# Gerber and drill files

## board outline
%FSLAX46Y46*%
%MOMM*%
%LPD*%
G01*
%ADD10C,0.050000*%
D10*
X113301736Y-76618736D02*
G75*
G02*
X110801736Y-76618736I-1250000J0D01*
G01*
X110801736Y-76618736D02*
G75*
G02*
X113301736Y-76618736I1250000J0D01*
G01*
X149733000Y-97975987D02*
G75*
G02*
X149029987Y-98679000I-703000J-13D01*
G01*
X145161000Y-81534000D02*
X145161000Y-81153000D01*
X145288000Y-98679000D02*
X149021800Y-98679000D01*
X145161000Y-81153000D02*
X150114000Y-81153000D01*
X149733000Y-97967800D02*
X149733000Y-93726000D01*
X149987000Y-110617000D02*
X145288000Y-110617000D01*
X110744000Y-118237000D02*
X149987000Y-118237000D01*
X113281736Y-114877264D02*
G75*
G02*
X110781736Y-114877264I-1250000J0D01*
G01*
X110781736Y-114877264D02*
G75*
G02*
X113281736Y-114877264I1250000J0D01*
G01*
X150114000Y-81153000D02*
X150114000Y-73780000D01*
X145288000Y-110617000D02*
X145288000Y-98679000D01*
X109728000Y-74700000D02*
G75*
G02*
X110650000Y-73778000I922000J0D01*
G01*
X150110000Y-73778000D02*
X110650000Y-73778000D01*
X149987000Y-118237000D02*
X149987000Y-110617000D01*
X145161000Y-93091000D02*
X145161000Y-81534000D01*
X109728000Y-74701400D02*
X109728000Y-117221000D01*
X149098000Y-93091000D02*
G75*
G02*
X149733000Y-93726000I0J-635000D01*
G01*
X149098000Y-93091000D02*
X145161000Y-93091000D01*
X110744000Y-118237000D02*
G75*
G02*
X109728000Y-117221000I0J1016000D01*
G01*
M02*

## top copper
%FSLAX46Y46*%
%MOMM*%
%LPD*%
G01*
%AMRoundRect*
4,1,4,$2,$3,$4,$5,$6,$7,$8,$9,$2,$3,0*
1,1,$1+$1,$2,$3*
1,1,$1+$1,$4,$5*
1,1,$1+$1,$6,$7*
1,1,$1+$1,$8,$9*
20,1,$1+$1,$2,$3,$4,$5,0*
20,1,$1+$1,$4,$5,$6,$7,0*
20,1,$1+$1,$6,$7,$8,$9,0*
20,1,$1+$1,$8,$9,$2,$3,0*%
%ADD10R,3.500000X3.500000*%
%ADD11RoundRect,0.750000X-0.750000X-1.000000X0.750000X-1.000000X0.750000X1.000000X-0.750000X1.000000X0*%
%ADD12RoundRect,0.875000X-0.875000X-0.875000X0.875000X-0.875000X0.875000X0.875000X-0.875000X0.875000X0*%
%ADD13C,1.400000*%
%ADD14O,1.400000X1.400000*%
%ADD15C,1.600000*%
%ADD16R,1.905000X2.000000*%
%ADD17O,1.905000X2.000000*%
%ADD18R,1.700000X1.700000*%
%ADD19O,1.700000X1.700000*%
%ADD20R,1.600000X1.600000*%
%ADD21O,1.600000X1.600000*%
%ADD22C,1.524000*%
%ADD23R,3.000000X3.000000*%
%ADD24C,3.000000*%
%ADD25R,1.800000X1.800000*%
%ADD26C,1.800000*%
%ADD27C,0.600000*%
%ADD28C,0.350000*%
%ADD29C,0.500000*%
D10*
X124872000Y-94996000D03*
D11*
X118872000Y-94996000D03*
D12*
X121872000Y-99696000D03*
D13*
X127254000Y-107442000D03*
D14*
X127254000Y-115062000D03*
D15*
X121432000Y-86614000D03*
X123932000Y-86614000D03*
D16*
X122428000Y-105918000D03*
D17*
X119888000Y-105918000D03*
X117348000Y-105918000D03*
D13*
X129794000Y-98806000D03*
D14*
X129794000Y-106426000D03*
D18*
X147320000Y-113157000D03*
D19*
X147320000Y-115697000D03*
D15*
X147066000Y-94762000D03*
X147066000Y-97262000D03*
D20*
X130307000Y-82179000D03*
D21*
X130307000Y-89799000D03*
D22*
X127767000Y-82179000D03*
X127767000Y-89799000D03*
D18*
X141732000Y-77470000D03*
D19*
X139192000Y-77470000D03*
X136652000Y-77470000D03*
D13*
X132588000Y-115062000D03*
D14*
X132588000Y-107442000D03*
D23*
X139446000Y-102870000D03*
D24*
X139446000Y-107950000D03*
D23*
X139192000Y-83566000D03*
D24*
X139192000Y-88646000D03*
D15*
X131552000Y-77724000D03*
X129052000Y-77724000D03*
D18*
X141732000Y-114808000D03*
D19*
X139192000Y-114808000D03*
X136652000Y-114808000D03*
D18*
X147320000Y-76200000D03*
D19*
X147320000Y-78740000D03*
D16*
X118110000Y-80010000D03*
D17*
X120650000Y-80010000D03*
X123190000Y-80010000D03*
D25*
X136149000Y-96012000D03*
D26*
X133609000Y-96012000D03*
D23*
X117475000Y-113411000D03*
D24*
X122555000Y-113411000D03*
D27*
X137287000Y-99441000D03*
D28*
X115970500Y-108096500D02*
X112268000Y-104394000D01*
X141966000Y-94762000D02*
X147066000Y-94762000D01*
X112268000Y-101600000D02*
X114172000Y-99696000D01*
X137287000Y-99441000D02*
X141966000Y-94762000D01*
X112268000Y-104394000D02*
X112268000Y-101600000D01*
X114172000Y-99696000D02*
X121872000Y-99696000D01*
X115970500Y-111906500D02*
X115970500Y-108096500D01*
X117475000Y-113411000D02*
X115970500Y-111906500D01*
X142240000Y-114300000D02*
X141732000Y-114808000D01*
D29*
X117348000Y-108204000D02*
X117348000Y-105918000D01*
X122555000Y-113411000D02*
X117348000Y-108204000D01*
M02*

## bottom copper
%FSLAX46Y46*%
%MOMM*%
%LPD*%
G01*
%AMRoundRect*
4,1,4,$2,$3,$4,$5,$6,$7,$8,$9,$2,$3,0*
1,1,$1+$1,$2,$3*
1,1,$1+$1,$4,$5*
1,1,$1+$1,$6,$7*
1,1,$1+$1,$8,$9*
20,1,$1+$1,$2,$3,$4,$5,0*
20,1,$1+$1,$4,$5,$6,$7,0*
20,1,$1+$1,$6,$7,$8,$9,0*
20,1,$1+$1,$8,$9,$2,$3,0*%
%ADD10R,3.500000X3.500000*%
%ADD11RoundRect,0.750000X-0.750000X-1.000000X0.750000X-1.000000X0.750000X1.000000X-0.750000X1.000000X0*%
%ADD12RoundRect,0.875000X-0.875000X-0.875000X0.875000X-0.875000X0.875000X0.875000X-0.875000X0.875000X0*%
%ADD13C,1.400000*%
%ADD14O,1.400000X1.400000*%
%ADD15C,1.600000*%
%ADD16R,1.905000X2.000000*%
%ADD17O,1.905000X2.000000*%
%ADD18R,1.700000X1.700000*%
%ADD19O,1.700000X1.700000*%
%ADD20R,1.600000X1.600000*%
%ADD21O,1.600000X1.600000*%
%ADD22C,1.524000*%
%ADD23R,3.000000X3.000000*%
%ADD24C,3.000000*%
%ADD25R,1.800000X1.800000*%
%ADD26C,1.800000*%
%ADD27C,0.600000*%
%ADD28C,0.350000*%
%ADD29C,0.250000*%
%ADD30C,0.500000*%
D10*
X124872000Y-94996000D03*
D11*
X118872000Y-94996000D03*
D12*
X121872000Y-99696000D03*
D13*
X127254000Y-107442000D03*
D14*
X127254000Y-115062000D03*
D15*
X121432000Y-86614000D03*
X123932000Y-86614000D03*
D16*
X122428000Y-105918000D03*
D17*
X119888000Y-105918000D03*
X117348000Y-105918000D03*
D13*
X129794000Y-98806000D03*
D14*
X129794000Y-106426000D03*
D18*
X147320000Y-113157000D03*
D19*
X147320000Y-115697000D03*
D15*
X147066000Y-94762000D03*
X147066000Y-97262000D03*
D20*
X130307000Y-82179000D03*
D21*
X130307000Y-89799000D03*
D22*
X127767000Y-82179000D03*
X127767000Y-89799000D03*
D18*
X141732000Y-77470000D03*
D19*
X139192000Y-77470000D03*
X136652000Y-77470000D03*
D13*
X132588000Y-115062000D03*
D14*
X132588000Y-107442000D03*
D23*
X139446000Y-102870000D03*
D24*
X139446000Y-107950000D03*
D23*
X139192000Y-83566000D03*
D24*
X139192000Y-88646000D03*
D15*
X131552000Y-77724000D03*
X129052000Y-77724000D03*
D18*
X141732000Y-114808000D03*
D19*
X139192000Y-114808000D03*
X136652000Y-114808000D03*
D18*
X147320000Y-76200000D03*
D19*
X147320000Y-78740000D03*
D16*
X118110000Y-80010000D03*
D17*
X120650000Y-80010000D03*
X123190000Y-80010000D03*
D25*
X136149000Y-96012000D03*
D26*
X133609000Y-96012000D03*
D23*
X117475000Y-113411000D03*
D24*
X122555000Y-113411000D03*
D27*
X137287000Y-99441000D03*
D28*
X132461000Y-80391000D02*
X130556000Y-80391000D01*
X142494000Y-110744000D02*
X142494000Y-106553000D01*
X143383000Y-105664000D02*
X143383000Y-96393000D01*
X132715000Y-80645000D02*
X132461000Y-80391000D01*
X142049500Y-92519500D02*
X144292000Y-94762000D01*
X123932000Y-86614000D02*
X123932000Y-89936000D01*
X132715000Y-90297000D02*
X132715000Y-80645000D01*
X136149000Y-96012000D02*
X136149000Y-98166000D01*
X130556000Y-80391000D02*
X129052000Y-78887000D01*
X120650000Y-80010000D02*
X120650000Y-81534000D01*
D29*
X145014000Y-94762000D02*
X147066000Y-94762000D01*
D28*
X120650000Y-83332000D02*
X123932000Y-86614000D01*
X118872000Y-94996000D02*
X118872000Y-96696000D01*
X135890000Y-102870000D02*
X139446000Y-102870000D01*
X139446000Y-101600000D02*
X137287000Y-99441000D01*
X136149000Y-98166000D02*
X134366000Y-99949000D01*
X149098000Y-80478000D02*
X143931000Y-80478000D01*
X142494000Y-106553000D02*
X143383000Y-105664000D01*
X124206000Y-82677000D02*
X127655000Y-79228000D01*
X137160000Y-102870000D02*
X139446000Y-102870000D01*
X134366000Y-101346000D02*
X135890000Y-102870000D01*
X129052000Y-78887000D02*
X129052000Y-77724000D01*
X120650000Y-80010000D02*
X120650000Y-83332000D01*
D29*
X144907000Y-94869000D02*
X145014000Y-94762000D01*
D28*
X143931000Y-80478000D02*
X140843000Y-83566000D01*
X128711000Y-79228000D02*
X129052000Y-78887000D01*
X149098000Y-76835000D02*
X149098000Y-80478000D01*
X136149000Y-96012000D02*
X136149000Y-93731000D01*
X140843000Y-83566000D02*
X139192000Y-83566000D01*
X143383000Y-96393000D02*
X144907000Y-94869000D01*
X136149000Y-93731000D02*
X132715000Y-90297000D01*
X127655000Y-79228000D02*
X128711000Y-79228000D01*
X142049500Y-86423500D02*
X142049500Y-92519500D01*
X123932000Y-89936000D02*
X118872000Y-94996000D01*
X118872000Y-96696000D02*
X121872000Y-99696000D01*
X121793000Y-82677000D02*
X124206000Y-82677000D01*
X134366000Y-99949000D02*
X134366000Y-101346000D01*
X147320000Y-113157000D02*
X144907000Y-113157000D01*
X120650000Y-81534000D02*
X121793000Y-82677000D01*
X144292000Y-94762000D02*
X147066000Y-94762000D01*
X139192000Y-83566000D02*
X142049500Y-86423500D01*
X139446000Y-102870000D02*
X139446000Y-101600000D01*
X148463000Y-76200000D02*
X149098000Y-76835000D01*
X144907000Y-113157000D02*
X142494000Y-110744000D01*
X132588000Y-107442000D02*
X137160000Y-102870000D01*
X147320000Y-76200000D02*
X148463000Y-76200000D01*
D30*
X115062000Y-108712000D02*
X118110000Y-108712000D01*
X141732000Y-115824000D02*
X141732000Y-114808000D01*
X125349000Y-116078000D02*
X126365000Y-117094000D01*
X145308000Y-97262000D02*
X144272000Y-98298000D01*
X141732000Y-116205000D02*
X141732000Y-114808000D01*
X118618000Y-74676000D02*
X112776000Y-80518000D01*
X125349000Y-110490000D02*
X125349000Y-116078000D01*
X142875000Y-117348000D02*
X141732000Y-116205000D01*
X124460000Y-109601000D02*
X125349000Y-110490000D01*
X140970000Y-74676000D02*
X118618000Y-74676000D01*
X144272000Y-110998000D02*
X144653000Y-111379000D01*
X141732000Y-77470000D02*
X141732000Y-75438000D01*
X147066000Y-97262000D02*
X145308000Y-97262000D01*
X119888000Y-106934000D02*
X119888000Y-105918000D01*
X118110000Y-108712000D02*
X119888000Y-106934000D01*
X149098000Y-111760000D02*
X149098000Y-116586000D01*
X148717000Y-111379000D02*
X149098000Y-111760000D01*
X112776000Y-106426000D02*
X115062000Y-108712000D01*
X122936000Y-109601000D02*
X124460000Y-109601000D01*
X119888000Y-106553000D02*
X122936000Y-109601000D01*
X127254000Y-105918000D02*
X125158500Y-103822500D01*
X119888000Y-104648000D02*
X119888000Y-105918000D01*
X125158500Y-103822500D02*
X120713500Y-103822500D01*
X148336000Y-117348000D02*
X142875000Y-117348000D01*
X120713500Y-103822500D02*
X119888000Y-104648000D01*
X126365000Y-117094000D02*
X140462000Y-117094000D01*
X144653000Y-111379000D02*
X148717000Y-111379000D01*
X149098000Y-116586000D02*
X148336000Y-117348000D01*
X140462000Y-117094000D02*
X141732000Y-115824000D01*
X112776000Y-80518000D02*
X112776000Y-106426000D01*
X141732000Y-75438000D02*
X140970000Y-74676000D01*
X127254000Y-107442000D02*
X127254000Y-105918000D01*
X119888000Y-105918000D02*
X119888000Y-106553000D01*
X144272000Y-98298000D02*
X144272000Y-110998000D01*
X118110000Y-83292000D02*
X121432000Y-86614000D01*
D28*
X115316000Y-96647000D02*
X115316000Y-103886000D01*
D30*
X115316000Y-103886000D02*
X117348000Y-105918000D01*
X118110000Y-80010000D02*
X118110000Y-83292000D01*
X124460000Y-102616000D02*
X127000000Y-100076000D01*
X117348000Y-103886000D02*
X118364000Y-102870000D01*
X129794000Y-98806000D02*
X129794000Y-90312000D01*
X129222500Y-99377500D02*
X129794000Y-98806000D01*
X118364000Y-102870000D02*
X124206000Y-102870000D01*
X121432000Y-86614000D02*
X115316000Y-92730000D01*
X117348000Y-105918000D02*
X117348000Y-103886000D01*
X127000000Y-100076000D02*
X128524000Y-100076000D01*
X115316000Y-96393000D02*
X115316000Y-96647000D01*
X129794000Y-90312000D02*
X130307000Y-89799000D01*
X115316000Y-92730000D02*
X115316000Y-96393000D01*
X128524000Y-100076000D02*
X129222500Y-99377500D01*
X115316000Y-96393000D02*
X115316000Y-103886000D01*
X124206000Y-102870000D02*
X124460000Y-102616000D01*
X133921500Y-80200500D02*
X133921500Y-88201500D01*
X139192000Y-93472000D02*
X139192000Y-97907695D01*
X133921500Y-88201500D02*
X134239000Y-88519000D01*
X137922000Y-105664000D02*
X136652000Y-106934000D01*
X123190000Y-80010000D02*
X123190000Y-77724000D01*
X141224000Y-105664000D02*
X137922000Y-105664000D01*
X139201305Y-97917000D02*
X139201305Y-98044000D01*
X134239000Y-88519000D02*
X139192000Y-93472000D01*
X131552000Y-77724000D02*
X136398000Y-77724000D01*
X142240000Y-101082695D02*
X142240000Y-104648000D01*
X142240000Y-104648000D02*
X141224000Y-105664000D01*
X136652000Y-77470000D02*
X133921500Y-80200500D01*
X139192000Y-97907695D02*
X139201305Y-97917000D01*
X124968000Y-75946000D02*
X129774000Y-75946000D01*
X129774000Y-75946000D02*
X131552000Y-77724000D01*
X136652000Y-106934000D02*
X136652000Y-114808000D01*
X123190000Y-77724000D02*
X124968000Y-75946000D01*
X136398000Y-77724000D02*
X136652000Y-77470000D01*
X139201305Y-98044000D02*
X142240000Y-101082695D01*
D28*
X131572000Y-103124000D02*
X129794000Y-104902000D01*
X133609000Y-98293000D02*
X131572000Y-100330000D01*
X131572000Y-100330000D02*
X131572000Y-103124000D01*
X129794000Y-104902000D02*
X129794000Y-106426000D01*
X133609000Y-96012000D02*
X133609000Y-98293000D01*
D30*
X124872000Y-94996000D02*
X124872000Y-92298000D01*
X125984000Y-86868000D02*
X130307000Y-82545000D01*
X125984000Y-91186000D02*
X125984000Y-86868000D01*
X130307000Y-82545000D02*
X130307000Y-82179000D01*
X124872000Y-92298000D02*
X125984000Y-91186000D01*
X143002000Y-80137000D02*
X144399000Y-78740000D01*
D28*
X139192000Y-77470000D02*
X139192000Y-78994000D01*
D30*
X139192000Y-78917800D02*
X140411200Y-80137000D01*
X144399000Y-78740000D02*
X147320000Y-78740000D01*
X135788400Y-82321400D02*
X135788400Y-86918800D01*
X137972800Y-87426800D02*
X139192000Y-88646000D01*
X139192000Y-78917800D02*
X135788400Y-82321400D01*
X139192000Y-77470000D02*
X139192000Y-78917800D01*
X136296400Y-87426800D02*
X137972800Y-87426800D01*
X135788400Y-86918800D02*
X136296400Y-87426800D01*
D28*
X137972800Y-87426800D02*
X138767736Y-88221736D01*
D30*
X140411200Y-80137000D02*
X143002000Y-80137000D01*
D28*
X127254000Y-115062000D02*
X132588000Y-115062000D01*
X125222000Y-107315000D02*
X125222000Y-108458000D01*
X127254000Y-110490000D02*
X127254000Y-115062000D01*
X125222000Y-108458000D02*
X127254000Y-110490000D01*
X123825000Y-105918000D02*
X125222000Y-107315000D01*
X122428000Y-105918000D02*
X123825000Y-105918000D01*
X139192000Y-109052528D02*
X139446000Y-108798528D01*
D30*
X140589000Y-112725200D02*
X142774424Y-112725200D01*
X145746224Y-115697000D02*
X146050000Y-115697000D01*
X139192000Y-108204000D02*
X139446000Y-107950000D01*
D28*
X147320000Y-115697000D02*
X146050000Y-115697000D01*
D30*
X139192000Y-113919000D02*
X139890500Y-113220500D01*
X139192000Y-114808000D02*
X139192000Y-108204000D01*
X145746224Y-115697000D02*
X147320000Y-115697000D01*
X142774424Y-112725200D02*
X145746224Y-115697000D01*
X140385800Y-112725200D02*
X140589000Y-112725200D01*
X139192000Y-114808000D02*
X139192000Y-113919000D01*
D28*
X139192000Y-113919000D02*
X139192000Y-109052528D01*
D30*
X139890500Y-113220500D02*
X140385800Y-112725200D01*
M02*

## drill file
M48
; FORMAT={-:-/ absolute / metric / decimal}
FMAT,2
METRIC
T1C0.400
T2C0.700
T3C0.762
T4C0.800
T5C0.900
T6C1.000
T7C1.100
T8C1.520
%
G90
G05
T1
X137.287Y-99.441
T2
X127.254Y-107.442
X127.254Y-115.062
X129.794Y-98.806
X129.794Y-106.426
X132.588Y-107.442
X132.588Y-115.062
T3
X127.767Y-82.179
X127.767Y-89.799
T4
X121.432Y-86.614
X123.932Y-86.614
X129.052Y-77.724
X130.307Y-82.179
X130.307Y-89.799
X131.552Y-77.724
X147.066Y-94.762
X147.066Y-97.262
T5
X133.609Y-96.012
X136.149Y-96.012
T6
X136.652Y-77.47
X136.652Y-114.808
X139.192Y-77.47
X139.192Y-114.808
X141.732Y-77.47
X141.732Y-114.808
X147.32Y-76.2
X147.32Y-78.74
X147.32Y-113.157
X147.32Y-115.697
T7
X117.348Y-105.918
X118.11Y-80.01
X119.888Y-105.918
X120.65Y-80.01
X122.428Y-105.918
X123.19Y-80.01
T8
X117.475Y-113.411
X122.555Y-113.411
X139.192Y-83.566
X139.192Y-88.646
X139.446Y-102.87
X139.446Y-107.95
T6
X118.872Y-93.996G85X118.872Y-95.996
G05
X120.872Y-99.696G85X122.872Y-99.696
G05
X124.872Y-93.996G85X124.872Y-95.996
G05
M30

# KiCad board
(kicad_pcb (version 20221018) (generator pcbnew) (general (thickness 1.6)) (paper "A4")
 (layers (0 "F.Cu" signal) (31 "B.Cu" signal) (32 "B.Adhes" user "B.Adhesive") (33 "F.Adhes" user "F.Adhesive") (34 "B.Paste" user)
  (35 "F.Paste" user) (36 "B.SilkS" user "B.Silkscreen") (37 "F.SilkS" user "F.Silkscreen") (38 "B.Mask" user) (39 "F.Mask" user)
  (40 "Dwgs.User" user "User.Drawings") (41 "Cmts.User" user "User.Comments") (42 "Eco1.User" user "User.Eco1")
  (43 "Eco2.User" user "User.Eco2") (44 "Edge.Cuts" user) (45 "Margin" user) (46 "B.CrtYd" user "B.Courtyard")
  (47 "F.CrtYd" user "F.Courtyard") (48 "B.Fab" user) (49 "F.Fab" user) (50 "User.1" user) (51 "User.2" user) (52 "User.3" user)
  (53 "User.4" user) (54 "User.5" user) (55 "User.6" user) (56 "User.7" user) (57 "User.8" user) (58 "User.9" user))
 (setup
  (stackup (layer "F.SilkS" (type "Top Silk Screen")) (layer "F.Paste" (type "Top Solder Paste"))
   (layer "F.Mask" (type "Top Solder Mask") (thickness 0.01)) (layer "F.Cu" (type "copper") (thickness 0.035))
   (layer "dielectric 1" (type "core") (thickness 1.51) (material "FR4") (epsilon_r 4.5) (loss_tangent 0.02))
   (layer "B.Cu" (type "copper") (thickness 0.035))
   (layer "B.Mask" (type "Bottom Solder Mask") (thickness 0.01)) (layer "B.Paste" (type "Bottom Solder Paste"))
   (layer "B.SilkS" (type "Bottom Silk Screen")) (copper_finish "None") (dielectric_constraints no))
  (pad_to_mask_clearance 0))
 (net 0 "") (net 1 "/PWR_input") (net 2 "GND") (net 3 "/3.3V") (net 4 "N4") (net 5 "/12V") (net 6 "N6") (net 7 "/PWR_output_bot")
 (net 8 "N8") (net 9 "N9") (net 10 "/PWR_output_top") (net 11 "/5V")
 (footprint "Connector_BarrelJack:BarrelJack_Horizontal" (layer "F.Cu") (at 124.872 94.996)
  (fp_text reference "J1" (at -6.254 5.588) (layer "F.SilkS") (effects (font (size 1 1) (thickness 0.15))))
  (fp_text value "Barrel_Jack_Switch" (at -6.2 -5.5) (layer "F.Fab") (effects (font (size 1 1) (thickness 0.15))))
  (pad "1" thru_hole rect (at 0 0) (size 3.5 3.5) (drill oval 1 3) (layers "*.Cu" "*.Mask") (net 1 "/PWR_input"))
  (pad "2" thru_hole roundrect (at -6 0) (size 3 3.5) (drill oval 1 3) (layers "*.Cu" "*.Mask") (roundrect_rratio 0.25) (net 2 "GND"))
  (pad "3" thru_hole roundrect (at -3 4.7) (size 3.5 3.5) (drill oval 3 1) (layers "*.Cu" "*.Mask") (roundrect_rratio 0.25) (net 2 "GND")))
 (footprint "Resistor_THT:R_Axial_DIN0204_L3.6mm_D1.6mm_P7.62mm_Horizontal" (layer "F.Cu") (at 127.254 107.442 -90)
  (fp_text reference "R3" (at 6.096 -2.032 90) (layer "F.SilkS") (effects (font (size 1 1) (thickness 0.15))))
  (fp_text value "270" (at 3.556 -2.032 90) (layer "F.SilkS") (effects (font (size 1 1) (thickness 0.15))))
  (pad "1" thru_hole circle (at 0 0 270) (size 1.4 1.4) (drill 0.7) (layers "*.Cu" "*.Mask") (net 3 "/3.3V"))
  (pad "2" thru_hole oval (at 7.62 0 270) (size 1.4 1.4) (drill 0.7) (layers "*.Cu" "*.Mask") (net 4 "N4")))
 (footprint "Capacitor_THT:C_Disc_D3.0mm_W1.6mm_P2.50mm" (layer "F.Cu") (at 121.432 86.614)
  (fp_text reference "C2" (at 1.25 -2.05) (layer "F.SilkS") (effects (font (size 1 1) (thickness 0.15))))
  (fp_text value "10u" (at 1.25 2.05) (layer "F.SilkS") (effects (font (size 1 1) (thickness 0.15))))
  (pad "1" thru_hole circle (at 0 0) (size 1.6 1.6) (drill 0.8) (layers "*.Cu" "*.Mask") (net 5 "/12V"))
  (pad "2" thru_hole circle (at 2.5 0) (size 1.6 1.6) (drill 0.8) (layers "*.Cu" "*.Mask") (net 2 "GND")))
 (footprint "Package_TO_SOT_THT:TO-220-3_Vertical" (layer "F.Cu") (at 122.428 105.918 180)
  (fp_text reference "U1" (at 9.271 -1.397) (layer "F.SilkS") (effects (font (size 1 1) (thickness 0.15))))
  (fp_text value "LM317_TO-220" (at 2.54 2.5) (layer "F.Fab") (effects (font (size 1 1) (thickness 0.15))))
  (pad "1" thru_hole rect (at 0 0 180) (size 1.905 2) (drill 1.1) (layers "*.Cu" "*.Mask") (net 4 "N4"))
  (pad "2" thru_hole oval (at 2.54 0 180) (size 1.905 2) (drill 1.1) (layers "*.Cu" "*.Mask") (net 3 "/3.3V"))
  (pad "3" thru_hole oval (at 5.08 0 180) (size 1.905 2) (drill 1.1) (layers "*.Cu" "*.Mask") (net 5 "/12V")))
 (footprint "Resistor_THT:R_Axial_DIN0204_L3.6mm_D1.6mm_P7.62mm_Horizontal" (layer "F.Cu") (at 129.794 98.806 -90)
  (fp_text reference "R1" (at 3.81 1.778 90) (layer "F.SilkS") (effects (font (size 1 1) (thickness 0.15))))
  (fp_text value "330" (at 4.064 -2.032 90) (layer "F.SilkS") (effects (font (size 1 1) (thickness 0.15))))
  (pad "1" thru_hole circle (at 0 0 270) (size 1.4 1.4) (drill 0.7) (layers "*.Cu" "*.Mask") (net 5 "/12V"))
  (pad "2" thru_hole oval (at 7.62 0 270) (size 1.4 1.4) (drill 0.7) (layers "*.Cu" "*.Mask") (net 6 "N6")))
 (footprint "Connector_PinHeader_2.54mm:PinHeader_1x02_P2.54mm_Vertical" (layer "F.Cu") (at 147.32 113.157)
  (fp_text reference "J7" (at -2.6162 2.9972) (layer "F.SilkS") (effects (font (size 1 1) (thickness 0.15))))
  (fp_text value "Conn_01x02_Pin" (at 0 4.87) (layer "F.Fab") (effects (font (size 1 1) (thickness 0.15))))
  (pad "1" thru_hole rect (at 0 0) (size 1.7 1.7) (drill 1) (layers "*.Cu" "*.Mask") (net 2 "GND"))
  (pad "2" thru_hole oval (at 0 2.54) (size 1.7 1.7) (drill 1) (layers "*.Cu" "*.Mask") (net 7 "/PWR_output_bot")))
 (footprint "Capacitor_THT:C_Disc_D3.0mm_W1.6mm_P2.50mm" (layer "F.Cu") (at 147.066 94.762 -90)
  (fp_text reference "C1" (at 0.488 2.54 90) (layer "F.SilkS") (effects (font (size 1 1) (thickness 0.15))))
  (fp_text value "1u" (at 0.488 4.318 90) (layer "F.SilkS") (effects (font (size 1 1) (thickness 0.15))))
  (pad "1" thru_hole circle (at 0 0 270) (size 1.6 1.6) (drill 0.8) (layers "*.Cu" "*.Mask") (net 2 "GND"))
  (pad "2" thru_hole circle (at 2.5 0 270) (size 1.6 1.6) (drill 0.8) (layers "*.Cu" "*.Mask") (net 3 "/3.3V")))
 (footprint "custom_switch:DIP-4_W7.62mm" (layer "F.Cu") (at 130.307 82.179 -90)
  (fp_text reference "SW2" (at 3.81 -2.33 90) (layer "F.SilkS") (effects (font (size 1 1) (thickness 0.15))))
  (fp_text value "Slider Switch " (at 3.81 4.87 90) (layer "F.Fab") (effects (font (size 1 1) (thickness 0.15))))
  (pad "1" thru_hole rect (at 0 0 270) (size 1.6 1.6) (drill 0.8) (layers "*.Cu" "*.Mask") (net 1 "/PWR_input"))
  (pad "2" thru_hole oval (at 7.62 0 270) (size 1.6 1.6) (drill 0.8) (layers "*.Cu" "*.Mask") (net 5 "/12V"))
  (pad "3" thru_hole circle (at 0 2.54 270) (size 1.524 1.524) (drill 0.762) (layers "*.Cu" "*.Mask") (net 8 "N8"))
  (pad "4" thru_hole circle (at 7.62 2.54 270) (size 1.524 1.524) (drill 0.762) (layers "*.Cu" "*.Mask") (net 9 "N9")))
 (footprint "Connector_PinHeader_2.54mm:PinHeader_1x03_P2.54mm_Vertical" (layer "F.Cu") (at 141.732 77.47 -90)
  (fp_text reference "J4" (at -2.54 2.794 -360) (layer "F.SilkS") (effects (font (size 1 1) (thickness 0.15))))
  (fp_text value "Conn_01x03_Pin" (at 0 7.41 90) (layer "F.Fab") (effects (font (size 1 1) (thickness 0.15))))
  (pad "1" thru_hole rect (at 0 0 270) (size 1.7 1.7) (drill 1) (layers "*.Cu" "*.Mask") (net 3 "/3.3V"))
  (pad "2" thru_hole oval (at 0 2.54 270) (size 1.7 1.7) (drill 1) (layers "*.Cu" "*.Mask") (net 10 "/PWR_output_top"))
  (pad "3" thru_hole oval (at 0 5.08 270) (size 1.7 1.7) (drill 1) (layers "*.Cu" "*.Mask") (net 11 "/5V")))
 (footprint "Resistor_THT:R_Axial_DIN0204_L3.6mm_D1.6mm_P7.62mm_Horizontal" (layer "F.Cu") (at 132.588 115.062 90)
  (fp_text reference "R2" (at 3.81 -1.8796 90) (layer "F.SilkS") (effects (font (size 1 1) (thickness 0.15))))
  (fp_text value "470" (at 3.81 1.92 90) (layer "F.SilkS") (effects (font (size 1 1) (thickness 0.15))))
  (pad "1" thru_hole circle (at 0 0 90) (size 1.4 1.4) (drill 0.7) (layers "*.Cu" "*.Mask") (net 4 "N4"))
  (pad "2" thru_hole oval (at 7.62 0 90) (size 1.4 1.4) (drill 0.7) (layers "*.Cu" "*.Mask") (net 2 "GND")))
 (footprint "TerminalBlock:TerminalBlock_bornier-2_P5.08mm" (layer "F.Cu") (at 139.446 102.87 -90)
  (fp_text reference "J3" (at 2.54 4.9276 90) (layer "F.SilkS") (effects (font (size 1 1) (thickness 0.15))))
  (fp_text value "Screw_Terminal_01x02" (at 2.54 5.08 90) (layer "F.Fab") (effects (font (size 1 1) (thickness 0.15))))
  (pad "1" thru_hole rect (at 0 0 270) (size 3 3) (drill 1.52) (layers "*.Cu" "*.Mask") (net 2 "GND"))
  (pad "2" thru_hole circle (at 5.08 0 270) (size 3 3) (drill 1.52) (layers "*.Cu" "*.Mask") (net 7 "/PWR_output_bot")))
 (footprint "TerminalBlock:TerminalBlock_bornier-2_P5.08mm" (layer "F.Cu") (at 139.192 83.566 -90)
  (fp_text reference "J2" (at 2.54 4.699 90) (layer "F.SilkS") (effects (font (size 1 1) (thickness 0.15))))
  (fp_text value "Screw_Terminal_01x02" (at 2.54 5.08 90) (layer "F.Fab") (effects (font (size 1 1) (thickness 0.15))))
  (pad "1" thru_hole rect (at 0 0 270) (size 3 3) (drill 1.52) (layers "*.Cu" "*.Mask") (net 2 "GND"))
  (pad "2" thru_hole circle (at 5.08 0 270) (size 3 3) (drill 1.52) (layers "*.Cu" "*.Mask") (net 10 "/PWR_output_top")))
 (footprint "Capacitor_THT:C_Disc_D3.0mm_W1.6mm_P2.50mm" (layer "F.Cu") (at 131.552 77.724 180)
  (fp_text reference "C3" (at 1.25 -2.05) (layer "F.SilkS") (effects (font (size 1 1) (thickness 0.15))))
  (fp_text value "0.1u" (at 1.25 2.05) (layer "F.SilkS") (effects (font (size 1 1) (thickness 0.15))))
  (pad "1" thru_hole circle (at 0 0 180) (size 1.6 1.6) (drill 0.8) (layers "*.Cu" "*.Mask") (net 11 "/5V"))
  (pad "2" thru_hole circle (at 2.5 0 180) (size 1.6 1.6) (drill 0.8) (layers "*.Cu" "*.Mask") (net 2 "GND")))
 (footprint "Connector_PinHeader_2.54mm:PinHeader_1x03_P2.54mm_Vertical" (layer "F.Cu") (at 141.732 114.808 -90)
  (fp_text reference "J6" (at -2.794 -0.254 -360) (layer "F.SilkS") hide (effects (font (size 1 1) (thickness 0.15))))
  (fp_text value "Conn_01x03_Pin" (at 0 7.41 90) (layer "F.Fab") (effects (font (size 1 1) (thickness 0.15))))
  (pad "1" thru_hole rect (at 0 0 270) (size 1.7 1.7) (drill 1) (layers "*.Cu" "*.Mask") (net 3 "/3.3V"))
  (pad "2" thru_hole oval (at 0 2.54 270) (size 1.7 1.7) (drill 1) (layers "*.Cu" "*.Mask") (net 7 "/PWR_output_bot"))
  (pad "3" thru_hole oval (at 0 5.08 270) (size 1.7 1.7) (drill 1) (layers "*.Cu" "*.Mask") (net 11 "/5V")))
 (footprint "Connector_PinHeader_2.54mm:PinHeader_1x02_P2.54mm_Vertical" (layer "F.Cu") (at 147.32 76.2)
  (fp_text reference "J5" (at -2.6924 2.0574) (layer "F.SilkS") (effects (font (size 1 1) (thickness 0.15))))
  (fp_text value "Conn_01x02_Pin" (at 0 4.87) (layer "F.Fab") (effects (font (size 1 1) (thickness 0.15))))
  (pad "1" thru_hole rect (at 0 0) (size 1.7 1.7) (drill 1) (layers "*.Cu" "*.Mask") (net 2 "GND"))
  (pad "2" thru_hole oval (at 0 2.54) (size 1.7 1.7) (drill 1) (layers "*.Cu" "*.Mask") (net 10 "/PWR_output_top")))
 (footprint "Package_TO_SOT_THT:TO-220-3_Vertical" (layer "F.Cu") (at 118.11 80.01)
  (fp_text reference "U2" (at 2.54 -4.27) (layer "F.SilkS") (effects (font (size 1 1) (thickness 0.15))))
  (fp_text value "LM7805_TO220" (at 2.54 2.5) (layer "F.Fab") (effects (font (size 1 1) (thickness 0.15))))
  (pad "1" thru_hole rect (at 0 0) (size 1.905 2) (drill 1.1) (layers "*.Cu" "*.Mask") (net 5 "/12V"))
  (pad "2" thru_hole oval (at 2.54 0) (size 1.905 2) (drill 1.1) (layers "*.Cu" "*.Mask") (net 2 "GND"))
  (pad "3" thru_hole oval (at 5.08 0) (size 1.905 2) (drill 1.1) (layers "*.Cu" "*.Mask") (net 11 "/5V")))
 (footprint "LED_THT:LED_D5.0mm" (layer "F.Cu") (at 136.149 96.012 180)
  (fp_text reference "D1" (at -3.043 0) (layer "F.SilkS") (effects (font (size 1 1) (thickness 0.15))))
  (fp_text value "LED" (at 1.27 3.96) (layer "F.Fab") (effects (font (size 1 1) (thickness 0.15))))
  (pad "1" thru_hole rect (at 0 0 180) (size 1.8 1.8) (drill 0.9) (layers "*.Cu" "*.Mask") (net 2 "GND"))
  (pad "2" thru_hole circle (at 2.54 0 180) (size 1.8 1.8) (drill 0.9) (layers "*.Cu" "*.Mask") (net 6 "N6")))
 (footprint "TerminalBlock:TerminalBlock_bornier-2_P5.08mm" (layer "F.Cu") (at 117.475 113.411)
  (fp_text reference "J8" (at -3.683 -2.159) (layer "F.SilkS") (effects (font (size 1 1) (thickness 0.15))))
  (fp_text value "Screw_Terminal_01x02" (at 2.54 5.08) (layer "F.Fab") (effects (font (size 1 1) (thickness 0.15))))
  (pad "1" thru_hole rect (at 0 0) (size 3 3) (drill 1.52) (layers "*.Cu" "*.Mask") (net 2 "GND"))
  (pad "2" thru_hole circle (at 5.08 0) (size 3 3) (drill 1.52) (layers "*.Cu" "*.Mask") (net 5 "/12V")))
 (gr_circle locked (center 112.051736 76.618736) (end 113.301736 76.618736) (stroke (width 0.05) (type default)) (fill none)
  (layer "Edge.Cuts"))
 (gr_arc locked (start 149.733 97.975987) (mid 149.527092 98.473092) (end 149.029987 98.679) (stroke (width 0.05) (type default))
  (layer "Edge.Cuts"))
 (gr_line locked (start 145.161 81.534) (end 145.161 81.153) (stroke (width 0.05) (type default)) (layer "Edge.Cuts"))
 (gr_line locked (start 145.288 98.679) (end 149.0218 98.679) (stroke (width 0.05) (type default)) (layer "Edge.Cuts"))
 (gr_line locked (start 145.161 81.153) (end 150.114 81.153) (stroke (width 0.05) (type default)) (layer "Edge.Cuts"))
 (gr_line locked (start 149.733 97.9678) (end 149.733 93.726) (stroke (width 0.05) (type default)) (layer "Edge.Cuts"))
 (gr_line locked (start 149.987 110.617) (end 145.288 110.617) (stroke (width 0.05) (type default)) (layer "Edge.Cuts"))
 (gr_line locked (start 110.744 118.237) (end 149.987 118.237) (stroke (width 0.05) (type default)) (layer "Edge.Cuts"))
 (gr_circle locked (center 112.031736 114.877264) (end 113.281736 114.877264) (stroke (width 0.05) (type default)) (fill none)
  (layer "Edge.Cuts"))
 (gr_line locked (start 150.114 81.153) (end 150.114 73.78) (stroke (width 0.05) (type default)) (layer "Edge.Cuts"))
 (gr_line locked (start 145.288 110.617) (end 145.288 98.679) (stroke (width 0.05) (type default)) (layer "Edge.Cuts"))
 (gr_arc locked (start 109.728 74.7) (mid 109.998048 74.048048) (end 110.65 73.778) (stroke (width 0.05) (type default)) (layer "Edge.Cuts"))
 (gr_line locked (start 150.11 73.778) (end 110.65 73.778) (stroke (width 0.05) (type default)) (layer "Edge.Cuts"))
 (gr_line locked (start 149.987 118.237) (end 149.987 110.617) (stroke (width 0.05) (type default)) (layer "Edge.Cuts"))
 (gr_line locked (start 145.161 93.091) (end 145.161 81.534) (stroke (width 0.05) (type default)) (layer "Edge.Cuts"))
 (gr_line locked (start 109.728 74.7014) (end 109.728 117.221) (stroke (width 0.05) (type default)) (layer "Edge.Cuts"))
 (gr_arc locked (start 149.098 93.091) (mid 149.547013 93.276987) (end 149.733 93.726) (stroke (width 0.05) (type default))
  (layer "Edge.Cuts"))
 (gr_line locked (start 149.098 93.091) (end 145.161 93.091) (stroke (width 0.05) (type default)) (layer "Edge.Cuts"))
 (gr_arc locked (start 110.744 118.237) (mid 110.02558 117.93942) (end 109.728 117.221) (stroke (width 0.05) (type default))
  (layer "Edge.Cuts"))
 (segment (start 115.9705 108.0965) (end 112.268 104.394) (width 0.35) (layer "F.Cu") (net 2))
 (segment (start 141.966 94.762) (end 147.066 94.762) (width 0.35) (layer "F.Cu") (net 2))
 (segment (start 112.268 101.6) (end 114.172 99.696) (width 0.35) (layer "F.Cu") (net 2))
 (segment (start 137.287 99.441) (end 141.966 94.762) (width 0.35) (layer "F.Cu") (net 2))
 (segment (start 112.268 104.394) (end 112.268 101.6) (width 0.35) (layer "F.Cu") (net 2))
 (segment (start 114.172 99.696) (end 121.872 99.696) (width 0.35) (layer "F.Cu") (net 2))
 (segment (start 115.9705 111.9065) (end 115.9705 108.0965) (width 0.35) (layer "F.Cu") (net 2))
 (segment (start 117.475 113.411) (end 115.9705 111.9065) (width 0.35) (layer "F.Cu") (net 2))
 (via (at 137.287 99.441) (size 0.6) (drill 0.4) (layers "F.Cu" "B.Cu") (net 2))
 (segment (start 132.461 80.391) (end 130.556 80.391) (width 0.35) (layer "B.Cu") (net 2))
 (segment (start 142.494 110.744) (end 142.494 106.553) (width 0.35) (layer "B.Cu") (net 2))
 (segment (start 143.383 105.664) (end 143.383 96.393) (width 0.35) (layer "B.Cu") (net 2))
 (segment (start 132.715 80.645) (end 132.461 80.391) (width 0.35) (layer "B.Cu") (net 2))
 (segment (start 142.0495 92.5195) (end 144.292 94.762) (width 0.35) (layer "B.Cu") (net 2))
 (segment (start 123.932 86.614) (end 123.932 89.936) (width 0.35) (layer "B.Cu") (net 2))
 (segment (start 132.715 90.297) (end 132.715 80.645) (width 0.35) (layer "B.Cu") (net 2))
 (segment (start 136.149 96.012) (end 136.149 98.166) (width 0.35) (layer "B.Cu") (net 2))
 (segment (start 130.556 80.391) (end 129.052 78.887) (width 0.35) (layer "B.Cu") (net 2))
 (segment (start 120.65 80.01) (end 120.65 81.534) (width 0.35) (layer "B.Cu") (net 2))
 (segment (start 145.014 94.762) (end 147.066 94.762) (width 0.25) (layer "B.Cu") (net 2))
 (segment (start 120.65 83.332) (end 123.932 86.614) (width 0.35) (layer "B.Cu") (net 2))
 (segment (start 118.872 94.996) (end 118.872 96.696) (width 0.35) (layer "B.Cu") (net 2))
 (segment (start 135.89 102.87) (end 139.446 102.87) (width 0.35) (layer "B.Cu") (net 2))
 (segment (start 139.446 101.6) (end 137.287 99.441) (width 0.35) (layer "B.Cu") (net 2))
 (segment (start 136.149 98.166) (end 134.366 99.949) (width 0.35) (layer "B.Cu") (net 2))
 (segment (start 149.098 80.478) (end 143.931 80.478) (width 0.35) (layer "B.Cu") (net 2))
 (segment (start 142.494 106.553) (end 143.383 105.664) (width 0.35) (layer "B.Cu") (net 2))
 (segment (start 124.206 82.677) (end 127.655 79.228) (width 0.35) (layer "B.Cu") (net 2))
 (segment (start 137.16 102.87) (end 139.446 102.87) (width 0.35) (layer "B.Cu") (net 2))
 (segment (start 134.366 101.346) (end 135.89 102.87) (width 0.35) (layer "B.Cu") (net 2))
 (segment (start 129.052 78.887) (end 129.052 77.724) (width 0.35) (layer "B.Cu") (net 2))
 (segment (start 120.65 80.01) (end 120.65 83.332) (width 0.35) (layer "B.Cu") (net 2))
 (segment (start 144.907 94.869) (end 145.014 94.762) (width 0.25) (layer "B.Cu") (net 2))
 (segment (start 143.931 80.478) (end 140.843 83.566) (width 0.35) (layer "B.Cu") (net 2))
 (segment (start 128.711 79.228) (end 129.052 78.887) (width 0.35) (layer "B.Cu") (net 2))
 (segment (start 149.098 76.835) (end 149.098 80.478) (width 0.35) (layer "B.Cu") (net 2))
 (segment (start 136.149 96.012) (end 136.149 93.731) (width 0.35) (layer "B.Cu") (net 2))
 (segment (start 140.843 83.566) (end 139.192 83.566) (width 0.35) (layer "B.Cu") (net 2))
 (segment (start 143.383 96.393) (end 144.907 94.869) (width 0.35) (layer "B.Cu") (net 2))
 (segment (start 136.149 93.731) (end 132.715 90.297) (width 0.35) (layer "B.Cu") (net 2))
 (segment (start 127.655 79.228) (end 128.711 79.228) (width 0.35) (layer "B.Cu") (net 2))
 (segment (start 142.0495 86.4235) (end 142.0495 92.5195) (width 0.35) (layer "B.Cu") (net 2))
 (segment (start 123.932 89.936) (end 118.872 94.996) (width 0.35) (layer "B.Cu") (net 2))
 (segment (start 118.872 96.696) (end 121.872 99.696) (width 0.35) (layer "B.Cu") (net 2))
 (segment (start 121.793 82.677) (end 124.206 82.677) (width 0.35) (layer "B.Cu") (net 2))
 (segment (start 134.366 99.949) (end 134.366 101.346) (width 0.35) (layer "B.Cu") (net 2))
 (segment (start 147.32 113.157) (end 144.907 113.157) (width 0.35) (layer "B.Cu") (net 2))
 (segment (start 120.65 81.534) (end 121.793 82.677) (width 0.35) (layer "B.Cu") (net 2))
 (segment (start 144.292 94.762) (end 147.066 94.762) (width 0.35) (layer "B.Cu") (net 2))
 (segment (start 139.192 83.566) (end 142.0495 86.4235) (width 0.35) (layer "B.Cu") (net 2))
 (segment (start 139.446 102.87) (end 139.446 101.6) (width 0.35) (layer "B.Cu") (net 2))
 (segment (start 148.463 76.2) (end 149.098 76.835) (width 0.35) (layer "B.Cu") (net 2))
 (segment (start 144.907 113.157) (end 142.494 110.744) (width 0.35) (layer "B.Cu") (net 2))
 (segment (start 132.588 107.442) (end 137.16 102.87) (width 0.35) (layer "B.Cu") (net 2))
 (segment (start 147.32 76.2) (end 148.463 76.2) (width 0.35) (layer "B.Cu") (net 2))
 (segment (start 142.24 114.3) (end 141.732 114.808) (width 0.35) (layer "F.Cu") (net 3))
 (segment (start 115.062 108.712) (end 118.11 108.712) (width 0.5) (layer "B.Cu") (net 3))
 (segment (start 141.732 115.824) (end 141.732 114.808) (width 0.5) (layer "B.Cu") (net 3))
 (segment (start 125.349 116.078) (end 126.365 117.094) (width 0.5) (layer "B.Cu") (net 3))
 (segment (start 145.308 97.262) (end 144.272 98.298) (width 0.5) (layer "B.Cu") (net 3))
 (segment (start 141.732 116.205) (end 141.732 114.808) (width 0.5) (layer "B.Cu") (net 3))
 (segment (start 118.618 74.676) (end 112.776 80.518) (width 0.5) (layer "B.Cu") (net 3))
 (segment (start 125.349 110.49) (end 125.349 116.078) (width 0.5) (layer "B.Cu") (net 3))
 (segment (start 142.875 117.348) (end 141.732 116.205) (width 0.5) (layer "B.Cu") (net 3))
 (segment (start 124.46 109.601) (end 125.349 110.49) (width 0.5) (layer "B.Cu") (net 3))
 (segment (start 140.97 74.676) (end 118.618 74.676) (width 0.5) (layer "B.Cu") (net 3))
 (segment (start 144.272 110.998) (end 144.653 111.379) (width 0.5) (layer "B.Cu") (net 3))
 (segment (start 141.732 77.47) (end 141.732 75.438) (width 0.5) (layer "B.Cu") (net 3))
 (segment (start 147.066 97.262) (end 145.308 97.262) (width 0.5) (layer "B.Cu") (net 3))
 (segment (start 119.888 106.934) (end 119.888 105.918) (width 0.5) (layer "B.Cu") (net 3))
 (segment (start 118.11 108.712) (end 119.888 106.934) (width 0.5) (layer "B.Cu") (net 3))
 (segment (start 149.098 111.76) (end 149.098 116.586) (width 0.5) (layer "B.Cu") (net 3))
 (segment (start 148.717 111.379) (end 149.098 111.76) (width 0.5) (layer "B.Cu") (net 3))
 (segment (start 112.776 106.426) (end 115.062 108.712) (width 0.5) (layer "B.Cu") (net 3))
 (segment (start 122.936 109.601) (end 124.46 109.601) (width 0.5) (layer "B.Cu") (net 3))
 (segment (start 119.888 106.553) (end 122.936 109.601) (width 0.5) (layer "B.Cu") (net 3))
 (segment (start 127.254 105.918) (end 125.1585 103.8225) (width 0.5) (layer "B.Cu") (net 3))
 (segment (start 119.888 104.648) (end 119.888 105.918) (width 0.5) (layer "B.Cu") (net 3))
 (segment (start 125.1585 103.8225) (end 120.7135 103.8225) (width 0.5) (layer "B.Cu") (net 3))
 (segment (start 148.336 117.348) (end 142.875 117.348) (width 0.5) (layer "B.Cu") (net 3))
 (segment (start 120.7135 103.8225) (end 119.888 104.648) (width 0.5) (layer "B.Cu") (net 3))
 (segment (start 126.365 117.094) (end 140.462 117.094) (width 0.5) (layer "B.Cu") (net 3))
 (segment (start 144.653 111.379) (end 148.717 111.379) (width 0.5) (layer "B.Cu") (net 3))
 (segment (start 149.098 116.586) (end 148.336 117.348) (width 0.5) (layer "B.Cu") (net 3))
 (segment (start 140.462 117.094) (end 141.732 115.824) (width 0.5) (layer "B.Cu") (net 3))
 (segment (start 112.776 80.518) (end 112.776 106.426) (width 0.5) (layer "B.Cu") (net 3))
 (segment (start 141.732 75.438) (end 140.97 74.676) (width 0.5) (layer "B.Cu") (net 3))
 (segment (start 127.254 107.442) (end 127.254 105.918) (width 0.5) (layer "B.Cu") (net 3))
 (segment (start 119.888 105.918) (end 119.888 106.553) (width 0.5) (layer "B.Cu") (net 3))
 (segment (start 144.272 98.298) (end 144.272 110.998) (width 0.5) (layer "B.Cu") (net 3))
 (segment (start 117.348 108.204) (end 117.348 105.918) (width 0.5) (layer "F.Cu") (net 5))
 (segment (start 122.555 113.411) (end 117.348 108.204) (width 0.5) (layer "F.Cu") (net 5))
 (segment (start 118.11 83.292) (end 121.432 86.614) (width 0.5) (layer "B.Cu") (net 5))
 (segment (start 115.316 96.647) (end 115.316 103.886) (width 0.35) (layer "B.Cu") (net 5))
 (segment (start 115.316 103.886) (end 117.348 105.918) (width 0.5) (layer "B.Cu") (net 5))
 (segment (start 118.11 80.01) (end 118.11 83.292) (width 0.5) (layer "B.Cu") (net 5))
 (segment (start 124.46 102.616) (end 127 100.076) (width 0.5) (layer "B.Cu") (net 5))
 (segment (start 117.348 103.886) (end 118.364 102.87) (width 0.5) (layer "B.Cu") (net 5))
 (segment (start 129.794 98.806) (end 129.794 90.312) (width 0.5) (layer "B.Cu") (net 5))
 (segment (start 129.2225 99.3775) (end 129.794 98.806) (width 0.5) (layer "B.Cu") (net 5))
 (segment (start 118.364 102.87) (end 124.206 102.87) (width 0.5) (layer "B.Cu") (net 5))
 (segment (start 121.432 86.614) (end 115.316 92.73) (width 0.5) (layer "B.Cu") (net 5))
 (segment (start 117.348 105.918) (end 117.348 103.886) (width 0.5) (layer "B.Cu") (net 5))
 (segment (start 127 100.076) (end 128.524 100.076) (width 0.5) (layer "B.Cu") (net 5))
 (segment (start 115.316 96.393) (end 115.316 96.647) (width 0.5) (layer "B.Cu") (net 5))
 (segment (start 129.794 90.312) (end 130.307 89.799) (width 0.5) (layer "B.Cu") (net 5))
 (segment (start 115.316 92.73) (end 115.316 96.393) (width 0.5) (layer "B.Cu") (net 5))
 (segment (start 128.524 100.076) (end 129.2225 99.3775) (width 0.5) (layer "B.Cu") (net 5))
 (segment (start 115.316 96.393) (end 115.316 103.886) (width 0.5) (layer "B.Cu") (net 5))
 (segment (start 124.206 102.87) (end 124.46 102.616) (width 0.5) (layer "B.Cu") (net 5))
 (segment (start 133.9215 80.2005) (end 133.9215 88.2015) (width 0.5) (layer "B.Cu") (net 11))
 (segment (start 139.192 93.472) (end 139.192 97.907695) (width 0.5) (layer "B.Cu") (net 11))
 (segment (start 133.9215 88.2015) (end 134.239 88.519) (width 0.5) (layer "B.Cu") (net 11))
 (segment (start 137.922 105.664) (end 136.652 106.934) (width 0.5) (layer "B.Cu") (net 11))
 (segment (start 123.19 80.01) (end 123.19 77.724) (width 0.5) (layer "B.Cu") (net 11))
 (segment (start 141.224 105.664) (end 137.922 105.664) (width 0.5) (layer "B.Cu") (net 11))
 (segment (start 139.201305 97.917) (end 139.201305 98.044) (width 0.5) (layer "B.Cu") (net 11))
 (segment (start 134.239 88.519) (end 139.192 93.472) (width 0.5) (layer "B.Cu") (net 11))
 (segment (start 131.552 77.724) (end 136.398 77.724) (width 0.5) (layer "B.Cu") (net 11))
 (segment (start 142.24 101.082695) (end 142.24 104.648) (width 0.5) (layer "B.Cu") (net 11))
 (segment (start 142.24 104.648) (end 141.224 105.664) (width 0.5) (layer "B.Cu") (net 11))
 (segment (start 136.652 77.47) (end 133.9215 80.2005) (width 0.5) (layer "B.Cu") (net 11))
 (segment (start 139.192 97.907695) (end 139.201305 97.917) (width 0.5) (layer "B.Cu") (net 11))
 (segment (start 124.968 75.946) (end 129.774 75.946) (width 0.5) (layer "B.Cu") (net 11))
 (segment (start 129.774 75.946) (end 131.552 77.724) (width 0.5) (layer "B.Cu") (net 11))
 (segment (start 136.652 106.934) (end 136.652 114.808) (width 0.5) (layer "B.Cu") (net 11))
 (segment (start 123.19 77.724) (end 124.968 75.946) (width 0.5) (layer "B.Cu") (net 11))
 (segment (start 136.398 77.724) (end 136.652 77.47) (width 0.5) (layer "B.Cu") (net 11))
 (segment (start 139.201305 98.044) (end 142.24 101.082695) (width 0.5) (layer "B.Cu") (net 11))
 (segment (start 131.572 103.124) (end 129.794 104.902) (width 0.35) (layer "B.Cu") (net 6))
 (segment (start 133.609 98.293) (end 131.572 100.33) (width 0.35) (layer "B.Cu") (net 6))
 (segment (start 131.572 100.33) (end 131.572 103.124) (width 0.35) (layer "B.Cu") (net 6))
 (segment (start 129.794 104.902) (end 129.794 106.426) (width 0.35) (layer "B.Cu") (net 6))
 (segment (start 133.609 96.012) (end 133.609 98.293) (width 0.35) (layer "B.Cu") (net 6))
 (segment (start 124.872 94.996) (end 124.872 92.298) (width 0.5) (layer "B.Cu") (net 1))
 (segment (start 125.984 86.868) (end 130.307 82.545) (width 0.5) (layer "B.Cu") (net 1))
 (segment (start 125.984 91.186) (end 125.984 86.868) (width 0.5) (layer "B.Cu") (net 1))
 (segment (start 130.307 82.545) (end 130.307 82.179) (width 0.5) (layer "B.Cu") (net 1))
 (segment (start 124.872 92.298) (end 125.984 91.186) (width 0.5) (layer "B.Cu") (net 1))
 (segment (start 143.002 80.137) (end 144.399 78.74) (width 0.5) (layer "B.Cu") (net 10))
 (segment (start 139.192 77.47) (end 139.192 78.994) (width 0.35) (layer "B.Cu") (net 10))
 (segment (start 139.192 78.9178) (end 140.4112 80.137) (width 0.5) (layer "B.Cu") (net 10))
 (segment (start 144.399 78.74) (end 147.32 78.74) (width 0.5) (layer "B.Cu") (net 10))
 (segment (start 135.7884 82.3214) (end 135.7884 86.9188) (width 0.5) (layer "B.Cu") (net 10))
 (segment (start 137.9728 87.4268) (end 139.192 88.646) (width 0.5) (layer "B.Cu") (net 10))
 (segment (start 139.192 78.9178) (end 135.7884 82.3214) (width 0.5) (layer "B.Cu") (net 10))
 (segment (start 139.192 77.47) (end 139.192 78.9178) (width 0.5) (layer "B.Cu") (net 10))
 (segment (start 136.2964 87.4268) (end 137.9728 87.4268) (width 0.5) (layer "B.Cu") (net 10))
 (segment (start 135.7884 86.9188) (end 136.2964 87.4268) (width 0.5) (layer "B.Cu") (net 10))
 (segment (start 137.9728 87.4268) (end 138.767736 88.221736) (width 0.35) (layer "B.Cu") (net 10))
 (segment (start 140.4112 80.137) (end 143.002 80.137) (width 0.5) (layer "B.Cu") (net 10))
 (segment (start 127.254 115.062) (end 132.588 115.062) (width 0.35) (layer "B.Cu") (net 4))
 (segment (start 125.222 107.315) (end 125.222 108.458) (width 0.35) (layer "B.Cu") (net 4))
 (segment (start 127.254 110.49) (end 127.254 115.062) (width 0.35) (layer "B.Cu") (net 4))
 (segment (start 125.222 108.458) (end 127.254 110.49) (width 0.35) (layer "B.Cu") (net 4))
 (segment (start 123.825 105.918) (end 125.222 107.315) (width 0.35) (layer "B.Cu") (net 4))
 (segment (start 122.428 105.918) (end 123.825 105.918) (width 0.35) (layer "B.Cu") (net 4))
 (segment (start 139.192 109.052528) (end 139.446 108.798528) (width 0.35) (layer "B.Cu") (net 7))
 (segment (start 140.589 112.7252) (end 142.774424 112.7252) (width 0.5) (layer "B.Cu") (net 7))
 (segment (start 145.746224 115.697) (end 146.05 115.697) (width 0.5) (layer "B.Cu") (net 7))
 (segment (start 139.192 108.204) (end 139.446 107.95) (width 0.5) (layer "B.Cu") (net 7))
 (segment (start 147.32 115.697) (end 146.05 115.697) (width 0.35) (layer "B.Cu") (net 7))
 (segment (start 139.192 113.919) (end 139.8905 113.2205) (width 0.5) (layer "B.Cu") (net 7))
 (segment (start 139.192 114.808) (end 139.192 108.204) (width 0.5) (layer "B.Cu") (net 7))
 (segment (start 145.746224 115.697) (end 147.32 115.697) (width 0.5) (layer "B.Cu") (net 7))
 (segment (start 142.774424 112.7252) (end 145.746224 115.697) (width 0.5) (layer "B.Cu") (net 7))
 (segment (start 140.3858 112.7252) (end 140.589 112.7252) (width 0.5) (layer "B.Cu") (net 7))
 (segment (start 139.192 114.808) (end 139.192 113.919) (width 0.5) (layer "B.Cu") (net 7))
 (segment (start 139.192 113.919) (end 139.192 109.052528) (width 0.35) (layer "B.Cu") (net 7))
 (segment (start 139.8905 113.2205) (end 140.3858 112.7252) (width 0.5) (layer "B.Cu") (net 7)))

